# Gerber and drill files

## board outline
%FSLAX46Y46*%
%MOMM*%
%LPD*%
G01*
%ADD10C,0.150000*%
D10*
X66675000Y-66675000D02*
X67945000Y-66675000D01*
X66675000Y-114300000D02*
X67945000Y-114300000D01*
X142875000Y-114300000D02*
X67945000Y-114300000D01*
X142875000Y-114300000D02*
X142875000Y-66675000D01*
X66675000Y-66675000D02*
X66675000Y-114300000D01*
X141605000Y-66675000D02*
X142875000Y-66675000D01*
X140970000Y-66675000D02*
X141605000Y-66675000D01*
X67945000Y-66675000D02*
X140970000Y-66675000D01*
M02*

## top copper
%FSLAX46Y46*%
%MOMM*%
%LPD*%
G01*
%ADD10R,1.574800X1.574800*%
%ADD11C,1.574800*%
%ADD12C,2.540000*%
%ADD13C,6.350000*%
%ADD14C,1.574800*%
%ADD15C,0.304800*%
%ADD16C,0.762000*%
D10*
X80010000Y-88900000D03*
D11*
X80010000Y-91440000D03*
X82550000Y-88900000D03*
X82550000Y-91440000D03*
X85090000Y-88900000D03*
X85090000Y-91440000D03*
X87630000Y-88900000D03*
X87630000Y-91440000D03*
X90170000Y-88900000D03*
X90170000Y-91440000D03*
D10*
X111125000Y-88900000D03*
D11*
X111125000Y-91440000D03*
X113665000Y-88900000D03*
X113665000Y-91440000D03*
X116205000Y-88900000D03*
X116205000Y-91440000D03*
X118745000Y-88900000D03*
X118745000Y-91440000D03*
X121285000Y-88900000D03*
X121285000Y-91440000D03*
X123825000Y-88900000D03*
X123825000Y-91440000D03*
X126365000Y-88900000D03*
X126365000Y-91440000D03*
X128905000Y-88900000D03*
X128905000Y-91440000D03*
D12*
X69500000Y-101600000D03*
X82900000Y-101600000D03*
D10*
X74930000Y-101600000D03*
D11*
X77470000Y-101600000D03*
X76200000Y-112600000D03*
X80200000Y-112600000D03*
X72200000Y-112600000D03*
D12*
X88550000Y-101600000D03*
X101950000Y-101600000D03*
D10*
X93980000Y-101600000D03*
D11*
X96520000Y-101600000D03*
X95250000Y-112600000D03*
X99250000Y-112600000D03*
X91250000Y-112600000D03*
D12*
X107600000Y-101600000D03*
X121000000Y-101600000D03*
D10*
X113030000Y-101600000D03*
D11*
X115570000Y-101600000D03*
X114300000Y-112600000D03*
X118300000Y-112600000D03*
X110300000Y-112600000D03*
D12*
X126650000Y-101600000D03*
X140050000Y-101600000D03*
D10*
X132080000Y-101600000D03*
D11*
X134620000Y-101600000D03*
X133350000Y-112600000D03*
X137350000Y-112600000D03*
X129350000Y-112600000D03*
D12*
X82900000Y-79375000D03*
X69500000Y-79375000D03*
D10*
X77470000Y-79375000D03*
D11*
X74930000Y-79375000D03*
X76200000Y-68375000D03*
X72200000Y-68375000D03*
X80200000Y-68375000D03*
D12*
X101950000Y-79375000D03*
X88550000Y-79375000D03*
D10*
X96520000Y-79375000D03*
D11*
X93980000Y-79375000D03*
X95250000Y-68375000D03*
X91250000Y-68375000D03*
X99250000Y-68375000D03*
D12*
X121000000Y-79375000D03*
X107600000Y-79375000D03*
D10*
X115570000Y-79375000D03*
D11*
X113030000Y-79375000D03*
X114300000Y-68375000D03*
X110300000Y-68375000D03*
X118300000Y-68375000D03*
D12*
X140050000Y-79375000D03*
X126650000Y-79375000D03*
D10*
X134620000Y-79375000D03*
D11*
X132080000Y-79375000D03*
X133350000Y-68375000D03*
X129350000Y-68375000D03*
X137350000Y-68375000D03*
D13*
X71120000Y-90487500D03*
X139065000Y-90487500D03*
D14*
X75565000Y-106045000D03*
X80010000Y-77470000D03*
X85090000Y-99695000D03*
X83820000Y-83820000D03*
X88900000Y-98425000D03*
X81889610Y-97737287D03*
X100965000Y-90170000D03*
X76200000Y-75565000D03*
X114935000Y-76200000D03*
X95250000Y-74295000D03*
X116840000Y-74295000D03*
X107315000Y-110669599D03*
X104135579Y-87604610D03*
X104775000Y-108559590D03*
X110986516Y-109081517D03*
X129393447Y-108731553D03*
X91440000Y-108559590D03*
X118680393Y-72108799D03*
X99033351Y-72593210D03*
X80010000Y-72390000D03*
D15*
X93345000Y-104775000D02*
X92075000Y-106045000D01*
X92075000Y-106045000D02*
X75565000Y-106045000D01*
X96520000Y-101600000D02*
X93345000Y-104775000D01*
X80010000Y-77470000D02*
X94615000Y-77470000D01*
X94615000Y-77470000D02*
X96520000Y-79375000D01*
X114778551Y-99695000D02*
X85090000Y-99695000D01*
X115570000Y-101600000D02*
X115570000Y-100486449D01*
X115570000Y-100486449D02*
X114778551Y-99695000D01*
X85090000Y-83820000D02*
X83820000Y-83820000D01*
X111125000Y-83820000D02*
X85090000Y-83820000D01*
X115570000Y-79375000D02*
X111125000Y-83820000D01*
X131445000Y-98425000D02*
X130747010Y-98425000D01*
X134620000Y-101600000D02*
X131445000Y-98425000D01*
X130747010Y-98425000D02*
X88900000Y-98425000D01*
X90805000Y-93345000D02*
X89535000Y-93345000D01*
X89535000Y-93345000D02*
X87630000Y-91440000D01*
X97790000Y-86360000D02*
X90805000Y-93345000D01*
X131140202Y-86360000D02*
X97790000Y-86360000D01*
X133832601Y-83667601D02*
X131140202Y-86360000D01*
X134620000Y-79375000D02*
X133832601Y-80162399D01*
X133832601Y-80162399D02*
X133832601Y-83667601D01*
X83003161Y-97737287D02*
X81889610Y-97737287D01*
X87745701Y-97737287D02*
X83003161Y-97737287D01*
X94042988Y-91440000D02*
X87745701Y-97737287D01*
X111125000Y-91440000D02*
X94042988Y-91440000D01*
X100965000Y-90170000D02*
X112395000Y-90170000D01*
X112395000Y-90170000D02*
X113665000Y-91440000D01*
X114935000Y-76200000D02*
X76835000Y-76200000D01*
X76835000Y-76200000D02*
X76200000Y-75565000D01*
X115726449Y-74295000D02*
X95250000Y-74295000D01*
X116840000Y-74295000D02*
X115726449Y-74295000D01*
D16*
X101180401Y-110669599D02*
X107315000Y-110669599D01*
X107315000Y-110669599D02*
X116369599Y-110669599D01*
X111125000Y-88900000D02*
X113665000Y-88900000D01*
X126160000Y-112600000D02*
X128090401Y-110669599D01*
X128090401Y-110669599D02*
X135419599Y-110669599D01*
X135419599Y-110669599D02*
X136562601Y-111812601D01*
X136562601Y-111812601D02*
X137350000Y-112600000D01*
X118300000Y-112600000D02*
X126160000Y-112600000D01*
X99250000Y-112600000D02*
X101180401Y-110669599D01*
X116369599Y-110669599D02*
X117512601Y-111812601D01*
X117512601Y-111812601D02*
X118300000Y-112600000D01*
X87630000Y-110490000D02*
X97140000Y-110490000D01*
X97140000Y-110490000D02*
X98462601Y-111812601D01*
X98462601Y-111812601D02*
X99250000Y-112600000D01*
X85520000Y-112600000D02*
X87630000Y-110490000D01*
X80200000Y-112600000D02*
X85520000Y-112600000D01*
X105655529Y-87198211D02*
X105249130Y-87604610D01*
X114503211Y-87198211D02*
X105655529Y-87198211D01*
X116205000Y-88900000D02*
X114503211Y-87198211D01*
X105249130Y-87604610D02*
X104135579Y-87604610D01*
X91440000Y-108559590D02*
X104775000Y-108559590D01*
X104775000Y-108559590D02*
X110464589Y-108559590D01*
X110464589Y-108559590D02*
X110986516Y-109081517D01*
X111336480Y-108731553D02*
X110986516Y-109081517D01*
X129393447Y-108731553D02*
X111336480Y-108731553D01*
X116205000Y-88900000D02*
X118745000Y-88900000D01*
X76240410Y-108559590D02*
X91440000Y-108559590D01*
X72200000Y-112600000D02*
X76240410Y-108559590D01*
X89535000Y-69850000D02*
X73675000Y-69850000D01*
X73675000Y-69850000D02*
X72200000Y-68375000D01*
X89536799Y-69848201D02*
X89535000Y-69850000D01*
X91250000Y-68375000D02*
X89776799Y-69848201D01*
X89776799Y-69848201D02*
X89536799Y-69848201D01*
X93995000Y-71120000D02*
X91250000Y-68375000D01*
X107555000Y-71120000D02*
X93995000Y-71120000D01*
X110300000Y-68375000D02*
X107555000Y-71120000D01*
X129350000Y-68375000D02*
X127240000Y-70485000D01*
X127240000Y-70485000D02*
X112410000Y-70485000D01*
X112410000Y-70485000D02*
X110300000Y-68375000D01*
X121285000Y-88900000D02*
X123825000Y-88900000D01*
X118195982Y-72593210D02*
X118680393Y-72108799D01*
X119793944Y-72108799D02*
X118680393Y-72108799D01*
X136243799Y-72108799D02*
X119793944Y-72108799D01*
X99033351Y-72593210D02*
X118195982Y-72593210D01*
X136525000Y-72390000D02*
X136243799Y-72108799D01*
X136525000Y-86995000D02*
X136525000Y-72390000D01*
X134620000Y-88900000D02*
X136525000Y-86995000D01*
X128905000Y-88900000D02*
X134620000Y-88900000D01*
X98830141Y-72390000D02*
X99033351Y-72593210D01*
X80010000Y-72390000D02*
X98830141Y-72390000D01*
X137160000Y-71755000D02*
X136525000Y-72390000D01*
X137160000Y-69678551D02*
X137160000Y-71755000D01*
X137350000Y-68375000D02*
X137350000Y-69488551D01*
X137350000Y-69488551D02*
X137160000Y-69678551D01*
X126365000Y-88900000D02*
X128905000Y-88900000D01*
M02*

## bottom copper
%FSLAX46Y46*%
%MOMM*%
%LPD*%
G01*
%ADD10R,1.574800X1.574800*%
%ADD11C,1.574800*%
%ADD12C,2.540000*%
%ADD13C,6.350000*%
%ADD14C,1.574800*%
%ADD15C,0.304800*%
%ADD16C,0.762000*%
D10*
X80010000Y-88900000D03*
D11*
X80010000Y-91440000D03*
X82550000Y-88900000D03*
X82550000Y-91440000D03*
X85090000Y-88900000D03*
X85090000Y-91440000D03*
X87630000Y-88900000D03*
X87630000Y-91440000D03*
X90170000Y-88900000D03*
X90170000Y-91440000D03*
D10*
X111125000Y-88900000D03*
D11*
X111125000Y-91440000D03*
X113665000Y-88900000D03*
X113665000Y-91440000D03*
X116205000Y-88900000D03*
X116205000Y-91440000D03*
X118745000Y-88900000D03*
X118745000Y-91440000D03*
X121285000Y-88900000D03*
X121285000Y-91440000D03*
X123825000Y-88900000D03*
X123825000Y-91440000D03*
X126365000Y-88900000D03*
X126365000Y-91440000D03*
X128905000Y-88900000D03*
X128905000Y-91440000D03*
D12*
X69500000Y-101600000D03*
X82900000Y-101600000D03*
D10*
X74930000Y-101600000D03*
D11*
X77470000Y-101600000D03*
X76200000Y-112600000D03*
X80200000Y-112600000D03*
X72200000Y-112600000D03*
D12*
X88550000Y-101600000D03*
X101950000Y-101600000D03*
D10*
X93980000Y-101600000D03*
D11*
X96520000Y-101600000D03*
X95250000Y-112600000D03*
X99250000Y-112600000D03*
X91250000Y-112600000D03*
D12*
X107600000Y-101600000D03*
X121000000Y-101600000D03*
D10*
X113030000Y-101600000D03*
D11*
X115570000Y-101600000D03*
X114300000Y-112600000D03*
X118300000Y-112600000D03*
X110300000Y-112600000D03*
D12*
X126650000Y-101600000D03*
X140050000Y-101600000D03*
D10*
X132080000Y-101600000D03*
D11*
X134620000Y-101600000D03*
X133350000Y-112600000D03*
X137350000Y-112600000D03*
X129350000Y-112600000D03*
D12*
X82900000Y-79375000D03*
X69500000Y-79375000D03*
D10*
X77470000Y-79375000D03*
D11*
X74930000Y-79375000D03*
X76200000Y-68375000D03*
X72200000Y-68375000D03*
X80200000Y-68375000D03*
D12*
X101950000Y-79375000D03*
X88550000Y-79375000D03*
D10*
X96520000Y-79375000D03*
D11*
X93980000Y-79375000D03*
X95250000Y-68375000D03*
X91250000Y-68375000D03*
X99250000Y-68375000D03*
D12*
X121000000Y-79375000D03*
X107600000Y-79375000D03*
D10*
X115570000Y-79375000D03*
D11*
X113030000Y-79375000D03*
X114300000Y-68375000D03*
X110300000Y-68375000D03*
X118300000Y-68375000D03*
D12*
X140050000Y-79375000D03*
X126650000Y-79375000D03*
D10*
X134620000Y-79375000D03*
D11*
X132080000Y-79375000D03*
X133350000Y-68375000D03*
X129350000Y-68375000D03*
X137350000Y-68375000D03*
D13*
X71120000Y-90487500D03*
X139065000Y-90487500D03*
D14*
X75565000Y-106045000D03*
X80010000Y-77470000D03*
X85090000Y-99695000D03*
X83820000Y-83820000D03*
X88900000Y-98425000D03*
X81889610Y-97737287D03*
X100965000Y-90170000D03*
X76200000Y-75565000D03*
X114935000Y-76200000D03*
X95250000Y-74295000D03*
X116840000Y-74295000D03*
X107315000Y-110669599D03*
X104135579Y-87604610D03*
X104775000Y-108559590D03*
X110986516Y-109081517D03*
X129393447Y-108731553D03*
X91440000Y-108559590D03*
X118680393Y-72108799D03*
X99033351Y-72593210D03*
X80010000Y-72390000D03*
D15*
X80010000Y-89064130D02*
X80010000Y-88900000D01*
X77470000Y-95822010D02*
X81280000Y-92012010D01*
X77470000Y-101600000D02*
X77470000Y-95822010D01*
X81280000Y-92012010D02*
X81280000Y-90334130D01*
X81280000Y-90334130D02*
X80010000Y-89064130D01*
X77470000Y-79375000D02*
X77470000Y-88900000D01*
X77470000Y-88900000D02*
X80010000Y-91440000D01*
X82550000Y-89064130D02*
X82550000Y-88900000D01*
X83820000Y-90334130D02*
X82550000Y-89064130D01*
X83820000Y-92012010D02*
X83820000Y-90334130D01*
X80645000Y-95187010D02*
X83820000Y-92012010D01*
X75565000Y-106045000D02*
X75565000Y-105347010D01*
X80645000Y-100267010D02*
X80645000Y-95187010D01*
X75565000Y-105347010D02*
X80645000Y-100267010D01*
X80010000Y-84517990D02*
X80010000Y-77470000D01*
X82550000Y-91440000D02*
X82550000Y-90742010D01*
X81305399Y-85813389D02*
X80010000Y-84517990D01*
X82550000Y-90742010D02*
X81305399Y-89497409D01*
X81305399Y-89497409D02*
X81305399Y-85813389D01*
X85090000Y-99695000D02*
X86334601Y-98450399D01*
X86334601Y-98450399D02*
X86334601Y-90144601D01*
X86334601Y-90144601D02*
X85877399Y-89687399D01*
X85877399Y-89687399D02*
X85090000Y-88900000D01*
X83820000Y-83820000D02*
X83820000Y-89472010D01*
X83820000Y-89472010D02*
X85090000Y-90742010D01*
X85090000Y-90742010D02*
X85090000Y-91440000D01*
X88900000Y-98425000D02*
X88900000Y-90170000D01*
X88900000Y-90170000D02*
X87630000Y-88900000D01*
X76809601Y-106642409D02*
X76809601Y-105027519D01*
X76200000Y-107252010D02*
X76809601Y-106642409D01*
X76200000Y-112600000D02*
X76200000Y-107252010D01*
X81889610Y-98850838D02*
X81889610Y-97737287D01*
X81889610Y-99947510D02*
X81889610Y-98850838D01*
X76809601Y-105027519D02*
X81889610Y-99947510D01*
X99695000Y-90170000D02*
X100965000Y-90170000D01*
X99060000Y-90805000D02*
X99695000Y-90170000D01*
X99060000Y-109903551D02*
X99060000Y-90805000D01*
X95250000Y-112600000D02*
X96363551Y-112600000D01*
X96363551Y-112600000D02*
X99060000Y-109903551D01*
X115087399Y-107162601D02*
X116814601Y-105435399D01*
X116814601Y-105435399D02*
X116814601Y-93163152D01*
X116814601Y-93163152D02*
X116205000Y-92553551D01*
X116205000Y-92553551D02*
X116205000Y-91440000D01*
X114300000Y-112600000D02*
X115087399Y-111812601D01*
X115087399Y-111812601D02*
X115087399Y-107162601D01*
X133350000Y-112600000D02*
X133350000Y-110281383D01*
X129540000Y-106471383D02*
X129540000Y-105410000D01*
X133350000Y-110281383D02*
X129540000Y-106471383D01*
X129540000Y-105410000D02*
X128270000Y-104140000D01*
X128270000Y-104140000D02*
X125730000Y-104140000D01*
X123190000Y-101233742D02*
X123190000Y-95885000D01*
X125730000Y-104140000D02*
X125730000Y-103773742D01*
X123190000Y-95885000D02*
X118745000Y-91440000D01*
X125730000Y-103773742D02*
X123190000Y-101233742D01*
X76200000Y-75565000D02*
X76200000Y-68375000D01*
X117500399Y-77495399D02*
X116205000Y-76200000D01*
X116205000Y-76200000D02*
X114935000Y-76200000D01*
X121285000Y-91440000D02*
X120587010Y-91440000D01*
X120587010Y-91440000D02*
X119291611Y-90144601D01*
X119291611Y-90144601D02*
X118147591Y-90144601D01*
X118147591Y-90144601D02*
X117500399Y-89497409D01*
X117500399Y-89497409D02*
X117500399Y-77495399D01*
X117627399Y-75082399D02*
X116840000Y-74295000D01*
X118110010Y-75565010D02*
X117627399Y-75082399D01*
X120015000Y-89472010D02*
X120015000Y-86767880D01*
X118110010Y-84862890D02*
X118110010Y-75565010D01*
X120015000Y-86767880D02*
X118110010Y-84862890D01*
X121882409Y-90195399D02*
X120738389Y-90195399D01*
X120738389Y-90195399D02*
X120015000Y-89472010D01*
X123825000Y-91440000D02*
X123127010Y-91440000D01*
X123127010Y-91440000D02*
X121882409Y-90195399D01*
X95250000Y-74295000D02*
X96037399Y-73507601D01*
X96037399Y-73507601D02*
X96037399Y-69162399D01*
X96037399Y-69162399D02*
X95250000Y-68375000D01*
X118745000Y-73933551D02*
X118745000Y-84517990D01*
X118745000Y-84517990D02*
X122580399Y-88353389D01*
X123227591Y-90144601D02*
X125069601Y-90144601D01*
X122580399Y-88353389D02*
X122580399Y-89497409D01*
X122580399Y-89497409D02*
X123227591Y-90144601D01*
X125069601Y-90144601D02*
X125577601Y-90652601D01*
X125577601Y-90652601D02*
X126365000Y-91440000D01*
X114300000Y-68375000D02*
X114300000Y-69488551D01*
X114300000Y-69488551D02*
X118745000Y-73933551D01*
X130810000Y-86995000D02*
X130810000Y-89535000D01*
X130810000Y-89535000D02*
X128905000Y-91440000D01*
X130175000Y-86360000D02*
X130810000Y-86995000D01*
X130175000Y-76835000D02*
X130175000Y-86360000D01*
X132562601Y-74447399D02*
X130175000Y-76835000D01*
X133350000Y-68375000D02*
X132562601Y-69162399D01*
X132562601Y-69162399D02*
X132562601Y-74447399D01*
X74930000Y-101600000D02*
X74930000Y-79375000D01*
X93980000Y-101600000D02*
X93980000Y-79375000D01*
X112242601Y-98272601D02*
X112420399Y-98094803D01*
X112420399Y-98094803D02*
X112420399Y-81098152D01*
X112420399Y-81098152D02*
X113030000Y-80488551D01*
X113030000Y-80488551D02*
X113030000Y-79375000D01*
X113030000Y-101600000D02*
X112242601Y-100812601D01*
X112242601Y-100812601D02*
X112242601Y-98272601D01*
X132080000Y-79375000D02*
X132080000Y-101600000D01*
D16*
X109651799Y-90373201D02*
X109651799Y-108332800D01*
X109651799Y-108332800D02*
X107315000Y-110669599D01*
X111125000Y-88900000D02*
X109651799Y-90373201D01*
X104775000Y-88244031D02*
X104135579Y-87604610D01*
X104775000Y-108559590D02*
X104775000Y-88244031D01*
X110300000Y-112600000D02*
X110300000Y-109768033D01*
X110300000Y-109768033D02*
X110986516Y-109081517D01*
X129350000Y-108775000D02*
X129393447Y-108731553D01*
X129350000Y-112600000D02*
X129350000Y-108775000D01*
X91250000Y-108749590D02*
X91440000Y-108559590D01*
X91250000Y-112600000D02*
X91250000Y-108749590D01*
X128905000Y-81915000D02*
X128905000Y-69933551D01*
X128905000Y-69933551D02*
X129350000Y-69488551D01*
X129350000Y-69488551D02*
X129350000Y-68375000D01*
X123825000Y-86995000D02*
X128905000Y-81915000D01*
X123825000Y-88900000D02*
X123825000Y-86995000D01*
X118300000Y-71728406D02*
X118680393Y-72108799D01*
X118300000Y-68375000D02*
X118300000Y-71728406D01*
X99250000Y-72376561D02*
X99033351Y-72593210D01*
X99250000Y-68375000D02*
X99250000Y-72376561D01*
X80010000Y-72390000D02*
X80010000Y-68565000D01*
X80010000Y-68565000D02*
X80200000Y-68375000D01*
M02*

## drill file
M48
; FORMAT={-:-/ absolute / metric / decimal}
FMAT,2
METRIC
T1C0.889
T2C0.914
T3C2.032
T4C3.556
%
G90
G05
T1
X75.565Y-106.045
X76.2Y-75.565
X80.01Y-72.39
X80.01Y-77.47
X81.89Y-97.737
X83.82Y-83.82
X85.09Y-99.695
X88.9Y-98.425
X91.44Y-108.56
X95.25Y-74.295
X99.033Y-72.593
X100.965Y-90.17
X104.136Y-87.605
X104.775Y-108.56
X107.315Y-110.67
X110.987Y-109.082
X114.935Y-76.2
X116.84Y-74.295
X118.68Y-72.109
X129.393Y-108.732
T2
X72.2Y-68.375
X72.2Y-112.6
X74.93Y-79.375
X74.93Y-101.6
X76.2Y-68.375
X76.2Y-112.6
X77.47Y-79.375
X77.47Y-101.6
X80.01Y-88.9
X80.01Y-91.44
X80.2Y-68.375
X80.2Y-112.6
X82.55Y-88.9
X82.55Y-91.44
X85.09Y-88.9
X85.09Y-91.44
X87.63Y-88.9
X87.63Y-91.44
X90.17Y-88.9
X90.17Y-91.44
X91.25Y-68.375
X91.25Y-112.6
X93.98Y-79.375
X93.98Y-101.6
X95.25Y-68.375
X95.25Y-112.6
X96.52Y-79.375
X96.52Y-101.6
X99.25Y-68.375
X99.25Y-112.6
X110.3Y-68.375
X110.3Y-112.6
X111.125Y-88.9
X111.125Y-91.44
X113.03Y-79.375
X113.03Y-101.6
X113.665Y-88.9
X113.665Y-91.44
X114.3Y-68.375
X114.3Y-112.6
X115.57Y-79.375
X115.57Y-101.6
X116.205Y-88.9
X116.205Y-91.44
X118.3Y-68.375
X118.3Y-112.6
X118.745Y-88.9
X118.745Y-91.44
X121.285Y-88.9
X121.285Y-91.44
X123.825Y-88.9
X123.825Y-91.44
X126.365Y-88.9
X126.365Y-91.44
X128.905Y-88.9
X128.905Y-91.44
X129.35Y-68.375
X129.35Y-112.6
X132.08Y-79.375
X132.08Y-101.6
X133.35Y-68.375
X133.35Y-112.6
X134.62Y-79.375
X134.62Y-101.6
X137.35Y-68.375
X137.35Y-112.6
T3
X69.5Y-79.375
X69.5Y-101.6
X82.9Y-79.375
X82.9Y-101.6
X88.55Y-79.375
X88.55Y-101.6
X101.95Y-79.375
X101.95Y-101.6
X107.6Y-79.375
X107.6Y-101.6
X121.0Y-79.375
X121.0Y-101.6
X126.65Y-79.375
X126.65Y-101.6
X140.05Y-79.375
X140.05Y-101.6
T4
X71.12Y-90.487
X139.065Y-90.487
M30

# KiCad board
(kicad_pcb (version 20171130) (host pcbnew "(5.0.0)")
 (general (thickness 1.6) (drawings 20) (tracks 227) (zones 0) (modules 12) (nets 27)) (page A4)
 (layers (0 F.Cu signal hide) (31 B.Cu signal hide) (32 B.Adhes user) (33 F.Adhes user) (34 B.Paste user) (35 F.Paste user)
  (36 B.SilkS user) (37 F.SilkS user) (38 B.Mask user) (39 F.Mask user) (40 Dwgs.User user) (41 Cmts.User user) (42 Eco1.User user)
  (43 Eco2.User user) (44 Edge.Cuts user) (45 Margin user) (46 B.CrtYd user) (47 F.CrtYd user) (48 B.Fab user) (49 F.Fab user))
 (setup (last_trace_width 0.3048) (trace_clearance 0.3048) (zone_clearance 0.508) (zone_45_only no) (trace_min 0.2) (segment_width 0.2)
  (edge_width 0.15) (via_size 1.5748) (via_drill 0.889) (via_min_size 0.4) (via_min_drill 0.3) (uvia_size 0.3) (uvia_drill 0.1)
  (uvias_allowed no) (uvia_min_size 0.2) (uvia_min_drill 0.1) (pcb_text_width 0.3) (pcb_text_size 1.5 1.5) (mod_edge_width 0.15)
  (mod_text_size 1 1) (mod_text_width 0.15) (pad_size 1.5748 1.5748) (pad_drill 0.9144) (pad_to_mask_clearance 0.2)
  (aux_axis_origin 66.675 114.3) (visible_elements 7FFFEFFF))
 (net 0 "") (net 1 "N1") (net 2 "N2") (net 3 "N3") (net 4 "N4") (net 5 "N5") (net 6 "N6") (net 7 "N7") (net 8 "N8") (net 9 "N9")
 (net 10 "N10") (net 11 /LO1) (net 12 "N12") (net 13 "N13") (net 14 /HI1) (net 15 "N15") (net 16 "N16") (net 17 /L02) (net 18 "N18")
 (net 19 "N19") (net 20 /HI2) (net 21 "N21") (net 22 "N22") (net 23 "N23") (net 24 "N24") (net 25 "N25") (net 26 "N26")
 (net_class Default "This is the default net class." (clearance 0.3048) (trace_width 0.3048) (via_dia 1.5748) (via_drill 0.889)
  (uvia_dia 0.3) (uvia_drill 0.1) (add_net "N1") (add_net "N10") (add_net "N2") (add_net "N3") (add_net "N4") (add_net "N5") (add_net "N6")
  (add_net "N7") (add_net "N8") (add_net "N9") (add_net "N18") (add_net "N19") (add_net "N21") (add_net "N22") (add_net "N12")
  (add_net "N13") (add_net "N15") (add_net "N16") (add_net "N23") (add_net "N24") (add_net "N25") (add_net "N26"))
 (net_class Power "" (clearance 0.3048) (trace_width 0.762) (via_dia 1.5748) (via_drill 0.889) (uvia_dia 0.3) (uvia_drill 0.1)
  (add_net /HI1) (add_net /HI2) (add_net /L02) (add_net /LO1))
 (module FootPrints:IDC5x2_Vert (layer B.Cu) (at 85.09 90.17 180)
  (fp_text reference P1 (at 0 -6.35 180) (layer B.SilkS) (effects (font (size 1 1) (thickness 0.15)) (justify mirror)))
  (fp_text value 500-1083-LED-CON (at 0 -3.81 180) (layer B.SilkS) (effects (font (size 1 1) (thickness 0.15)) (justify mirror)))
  (pad 1 thru_hole rect (at 5.08 1.27 180) (size 1.5748 1.5748) (drill 0.9144) (layers *.Cu *.Mask B.SilkS) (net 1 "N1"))
  (pad 2 thru_hole circle (at 5.08 -1.27 180) (size 1.5748 1.5748) (drill 0.9144) (layers *.Cu *.Mask B.SilkS) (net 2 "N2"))
  (pad 3 thru_hole circle (at 2.54 1.27 180) (size 1.5748 1.5748) (drill 0.9144) (layers *.Cu *.Mask B.SilkS) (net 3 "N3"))
  (pad 4 thru_hole circle (at 2.54 -1.27 180) (size 1.5748 1.5748) (drill 0.9144) (layers *.Cu *.Mask B.SilkS) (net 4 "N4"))
  (pad 5 thru_hole circle (at 0 1.27 180) (size 1.5748 1.5748) (drill 0.9144) (layers *.Cu *.Mask B.SilkS) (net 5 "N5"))
  (pad 6 thru_hole circle (at 0 -1.27 180) (size 1.5748 1.5748) (drill 0.9144) (layers *.Cu *.Mask B.SilkS) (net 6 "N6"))
  (pad 7 thru_hole circle (at -2.54 1.27 180) (size 1.5748 1.5748) (drill 0.9144) (layers *.Cu *.Mask B.SilkS) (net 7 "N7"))
  (pad 8 thru_hole circle (at -2.54 -1.27 180) (size 1.5748 1.5748) (drill 0.9144) (layers *.Cu *.Mask B.SilkS) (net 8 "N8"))
  (pad 9 thru_hole circle (at -5.08 1.27 180) (size 1.5748 1.5748) (drill 0.9144) (layers *.Cu *.Mask B.SilkS) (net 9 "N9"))
  (pad 10 thru_hole circle (at -5.08 -1.27 180) (size 1.5748 1.5748) (drill 0.9144) (layers *.Cu *.Mask B.SilkS) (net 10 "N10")))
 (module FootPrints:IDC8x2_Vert (layer B.Cu) (at 120.015 90.17 180)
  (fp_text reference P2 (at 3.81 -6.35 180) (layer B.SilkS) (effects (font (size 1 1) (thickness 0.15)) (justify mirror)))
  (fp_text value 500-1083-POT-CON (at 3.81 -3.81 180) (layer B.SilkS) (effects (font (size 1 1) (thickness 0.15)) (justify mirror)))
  (pad 1 thru_hole rect (at 8.89 1.27 180) (size 1.5748 1.5748) (drill 0.9144) (layers *.Cu *.Mask B.SilkS) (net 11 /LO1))
  (pad 2 thru_hole circle (at 8.89 -1.27 180) (size 1.5748 1.5748) (drill 0.9144) (layers *.Cu *.Mask B.SilkS) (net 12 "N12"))
  (pad 3 thru_hole circle (at 6.35 1.27 180) (size 1.5748 1.5748) (drill 0.9144) (layers *.Cu *.Mask B.SilkS) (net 11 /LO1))
  (pad 4 thru_hole circle (at 6.35 -1.27 180) (size 1.5748 1.5748) (drill 0.9144) (layers *.Cu *.Mask B.SilkS) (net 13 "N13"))
  (pad 5 thru_hole circle (at 3.81 1.27 180) (size 1.5748 1.5748) (drill 0.9144) (layers *.Cu *.Mask B.SilkS) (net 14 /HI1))
  (pad 6 thru_hole circle (at 3.81 -1.27 180) (size 1.5748 1.5748) (drill 0.9144) (layers *.Cu *.Mask B.SilkS) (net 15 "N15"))
  (pad 7 thru_hole circle (at 1.27 1.27 180) (size 1.5748 1.5748) (drill 0.9144) (layers *.Cu *.Mask B.SilkS) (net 14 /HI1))
  (pad 8 thru_hole circle (at 1.27 -1.27 180) (size 1.5748 1.5748) (drill 0.9144) (layers *.Cu *.Mask B.SilkS) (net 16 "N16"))
  (pad 9 thru_hole circle (at -1.27 1.27 180) (size 1.5748 1.5748) (drill 0.9144) (layers *.Cu *.Mask B.SilkS) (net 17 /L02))
  (pad 10 thru_hole circle (at -1.27 -1.27 180) (size 1.5748 1.5748) (drill 0.9144) (layers *.Cu *.Mask B.SilkS) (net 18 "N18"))
  (pad 11 thru_hole circle (at -3.81 1.27 180) (size 1.5748 1.5748) (drill 0.9144) (layers *.Cu *.Mask B.SilkS) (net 17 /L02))
  (pad 12 thru_hole circle (at -3.81 -1.27 180) (size 1.5748 1.5748) (drill 0.9144) (layers *.Cu *.Mask B.SilkS) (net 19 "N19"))
  (pad 13 thru_hole circle (at -6.35 1.27 180) (size 1.5748 1.5748) (drill 0.9144) (layers *.Cu *.Mask B.SilkS) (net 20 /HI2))
  (pad 14 thru_hole circle (at -6.35 -1.27 180) (size 1.5748 1.5748) (drill 0.9144) (layers *.Cu *.Mask B.SilkS) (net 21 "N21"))
  (pad 15 thru_hole circle (at -8.89 1.27 180) (size 1.5748 1.5748) (drill 0.9144) (layers *.Cu *.Mask B.SilkS) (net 20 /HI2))
  (pad 16 thru_hole circle (at -8.89 -1.27 180) (size 1.5748 1.5748) (drill 0.9144) (layers *.Cu *.Mask B.SilkS) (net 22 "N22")))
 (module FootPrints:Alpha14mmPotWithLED (layer F.Cu) (at 76.2 101.6)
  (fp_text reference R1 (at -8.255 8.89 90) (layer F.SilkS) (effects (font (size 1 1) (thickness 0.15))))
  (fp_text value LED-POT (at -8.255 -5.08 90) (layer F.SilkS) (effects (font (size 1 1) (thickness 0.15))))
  (pad "" thru_hole circle (at -6.7 0) (size 2.54 2.54) (drill 2.032) (layers *.Cu *.Mask F.SilkS))
  (pad "" thru_hole circle (at 6.7 0) (size 2.54 2.54) (drill 2.032) (layers *.Cu *.Mask F.SilkS))
  (pad 4 thru_hole rect (at -1.27 0) (size 1.5748 1.5748) (drill 0.9144) (layers *.Cu *.Mask F.SilkS) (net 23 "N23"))
  (pad 5 thru_hole circle (at 1.27 0) (size 1.5748 1.5748) (drill 0.9144) (layers *.Cu *.Mask F.SilkS) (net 1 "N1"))
  (pad 2 thru_hole circle (at 0 11) (size 1.5748 1.5748) (drill 0.9144) (layers *.Cu *.Mask F.SilkS) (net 12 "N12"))
  (pad 3 thru_hole circle (at 4 11) (size 1.5748 1.5748) (drill 0.9144) (layers *.Cu *.Mask F.SilkS) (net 11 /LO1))
  (pad 1 thru_hole circle (at -4 11) (size 1.5748 1.5748) (drill 0.9144) (layers *.Cu *.Mask F.SilkS) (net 14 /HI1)))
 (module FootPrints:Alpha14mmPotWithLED (layer F.Cu) (at 95.25 101.6)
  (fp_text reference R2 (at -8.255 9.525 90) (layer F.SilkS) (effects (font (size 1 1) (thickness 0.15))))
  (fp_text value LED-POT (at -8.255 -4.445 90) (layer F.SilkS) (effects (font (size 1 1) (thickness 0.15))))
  (pad "" thru_hole circle (at -6.7 0) (size 2.54 2.54) (drill 2.032) (layers *.Cu *.Mask F.SilkS))
  (pad "" thru_hole circle (at 6.7 0) (size 2.54 2.54) (drill 2.032) (layers *.Cu *.Mask F.SilkS))
  (pad 4 thru_hole rect (at -1.27 0) (size 1.5748 1.5748) (drill 0.9144) (layers *.Cu *.Mask F.SilkS) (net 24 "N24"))
  (pad 5 thru_hole circle (at 1.27 0) (size 1.5748 1.5748) (drill 0.9144) (layers *.Cu *.Mask F.SilkS) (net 3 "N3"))
  (pad 2 thru_hole circle (at 0 11) (size 1.5748 1.5748) (drill 0.9144) (layers *.Cu *.Mask F.SilkS) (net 13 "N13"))
  (pad 3 thru_hole circle (at 4 11) (size 1.5748 1.5748) (drill 0.9144) (layers *.Cu *.Mask F.SilkS) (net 11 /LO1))
  (pad 1 thru_hole circle (at -4 11) (size 1.5748 1.5748) (drill 0.9144) (layers *.Cu *.Mask F.SilkS) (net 14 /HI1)))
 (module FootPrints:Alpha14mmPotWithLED (layer F.Cu) (at 114.3 101.6)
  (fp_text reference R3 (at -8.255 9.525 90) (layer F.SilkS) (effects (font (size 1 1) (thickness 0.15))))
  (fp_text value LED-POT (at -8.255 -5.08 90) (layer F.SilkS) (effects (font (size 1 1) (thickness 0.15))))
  (pad "" thru_hole circle (at -6.7 0) (size 2.54 2.54) (drill 2.032) (layers *.Cu *.Mask F.SilkS))
  (pad "" thru_hole circle (at 6.7 0) (size 2.54 2.54) (drill 2.032) (layers *.Cu *.Mask F.SilkS))
  (pad 4 thru_hole rect (at -1.27 0) (size 1.5748 1.5748) (drill 0.9144) (layers *.Cu *.Mask F.SilkS) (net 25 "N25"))
  (pad 5 thru_hole circle (at 1.27 0) (size 1.5748 1.5748) (drill 0.9144) (layers *.Cu *.Mask F.SilkS) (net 5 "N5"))
  (pad 2 thru_hole circle (at 0 11) (size 1.5748 1.5748) (drill 0.9144) (layers *.Cu *.Mask F.SilkS) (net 15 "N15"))
  (pad 3 thru_hole circle (at 4 11) (size 1.5748 1.5748) (drill 0.9144) (layers *.Cu *.Mask F.SilkS) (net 11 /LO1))
  (pad 1 thru_hole circle (at -4 11) (size 1.5748 1.5748) (drill 0.9144) (layers *.Cu *.Mask F.SilkS) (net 14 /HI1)))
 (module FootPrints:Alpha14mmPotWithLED (layer F.Cu) (at 133.35 101.6)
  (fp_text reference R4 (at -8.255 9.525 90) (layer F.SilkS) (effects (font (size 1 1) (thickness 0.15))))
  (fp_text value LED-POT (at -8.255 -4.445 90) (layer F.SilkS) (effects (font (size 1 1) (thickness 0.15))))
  (pad "" thru_hole circle (at -6.7 0) (size 2.54 2.54) (drill 2.032) (layers *.Cu *.Mask F.SilkS))
  (pad "" thru_hole circle (at 6.7 0) (size 2.54 2.54) (drill 2.032) (layers *.Cu *.Mask F.SilkS))
  (pad 4 thru_hole rect (at -1.27 0) (size 1.5748 1.5748) (drill 0.9144) (layers *.Cu *.Mask F.SilkS) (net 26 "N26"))
  (pad 5 thru_hole circle (at 1.27 0) (size 1.5748 1.5748) (drill 0.9144) (layers *.Cu *.Mask F.SilkS) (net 7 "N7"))
  (pad 2 thru_hole circle (at 0 11) (size 1.5748 1.5748) (drill 0.9144) (layers *.Cu *.Mask F.SilkS) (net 16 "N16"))
  (pad 3 thru_hole circle (at 4 11) (size 1.5748 1.5748) (drill 0.9144) (layers *.Cu *.Mask F.SilkS) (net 11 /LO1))
  (pad 1 thru_hole circle (at -4 11) (size 1.5748 1.5748) (drill 0.9144) (layers *.Cu *.Mask F.SilkS) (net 14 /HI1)))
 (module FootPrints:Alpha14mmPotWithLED (layer F.Cu) (at 76.2 79.375 180)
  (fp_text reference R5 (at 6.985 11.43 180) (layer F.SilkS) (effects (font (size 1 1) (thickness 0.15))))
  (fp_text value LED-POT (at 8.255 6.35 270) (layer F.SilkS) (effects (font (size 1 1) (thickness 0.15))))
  (pad "" thru_hole circle (at -6.7 0 180) (size 2.54 2.54) (drill 2.032) (layers *.Cu *.Mask F.SilkS))
  (pad "" thru_hole circle (at 6.7 0 180) (size 2.54 2.54) (drill 2.032) (layers *.Cu *.Mask F.SilkS))
  (pad 4 thru_hole rect (at -1.27 0 180) (size 1.5748 1.5748) (drill 0.9144) (layers *.Cu *.Mask F.SilkS) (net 2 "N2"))
  (pad 5 thru_hole circle (at 1.27 0 180) (size 1.5748 1.5748) (drill 0.9144) (layers *.Cu *.Mask F.SilkS) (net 23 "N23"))
  (pad 2 thru_hole circle (at 0 11 180) (size 1.5748 1.5748) (drill 0.9144) (layers *.Cu *.Mask F.SilkS) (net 18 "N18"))
  (pad 3 thru_hole circle (at 4 11 180) (size 1.5748 1.5748) (drill 0.9144) (layers *.Cu *.Mask F.SilkS) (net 17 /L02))
  (pad 1 thru_hole circle (at -4 11 180) (size 1.5748 1.5748) (drill 0.9144) (layers *.Cu *.Mask F.SilkS) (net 20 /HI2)))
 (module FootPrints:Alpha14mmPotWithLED (layer F.Cu) (at 95.25 79.375 180)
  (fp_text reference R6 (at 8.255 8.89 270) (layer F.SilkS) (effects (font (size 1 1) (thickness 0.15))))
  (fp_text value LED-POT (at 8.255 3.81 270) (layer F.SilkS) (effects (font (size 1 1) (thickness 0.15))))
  (pad "" thru_hole circle (at -6.7 0 180) (size 2.54 2.54) (drill 2.032) (layers *.Cu *.Mask F.SilkS))
  (pad "" thru_hole circle (at 6.7 0 180) (size 2.54 2.54) (drill 2.032) (layers *.Cu *.Mask F.SilkS))
  (pad 4 thru_hole rect (at -1.27 0 180) (size 1.5748 1.5748) (drill 0.9144) (layers *.Cu *.Mask F.SilkS) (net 4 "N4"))
  (pad 5 thru_hole circle (at 1.27 0 180) (size 1.5748 1.5748) (drill 0.9144) (layers *.Cu *.Mask F.SilkS) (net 24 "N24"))
  (pad 2 thru_hole circle (at 0 11 180) (size 1.5748 1.5748) (drill 0.9144) (layers *.Cu *.Mask F.SilkS) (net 19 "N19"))
  (pad 3 thru_hole circle (at 4 11 180) (size 1.5748 1.5748) (drill 0.9144) (layers *.Cu *.Mask F.SilkS) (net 17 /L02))
  (pad 1 thru_hole circle (at -4 11 180) (size 1.5748 1.5748) (drill 0.9144) (layers *.Cu *.Mask F.SilkS) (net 20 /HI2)))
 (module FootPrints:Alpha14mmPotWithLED (layer F.Cu) (at 114.3 79.375 180)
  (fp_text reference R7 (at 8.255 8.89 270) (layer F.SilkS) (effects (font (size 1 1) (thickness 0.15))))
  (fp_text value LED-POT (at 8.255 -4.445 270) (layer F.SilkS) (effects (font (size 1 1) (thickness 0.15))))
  (pad "" thru_hole circle (at -6.7 0 180) (size 2.54 2.54) (drill 2.032) (layers *.Cu *.Mask F.SilkS))
  (pad "" thru_hole circle (at 6.7 0 180) (size 2.54 2.54) (drill 2.032) (layers *.Cu *.Mask F.SilkS))
  (pad 4 thru_hole rect (at -1.27 0 180) (size 1.5748 1.5748) (drill 0.9144) (layers *.Cu *.Mask F.SilkS) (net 6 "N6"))
  (pad 5 thru_hole circle (at 1.27 0 180) (size 1.5748 1.5748) (drill 0.9144) (layers *.Cu *.Mask F.SilkS) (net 25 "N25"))
  (pad 2 thru_hole circle (at 0 11 180) (size 1.5748 1.5748) (drill 0.9144) (layers *.Cu *.Mask F.SilkS) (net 21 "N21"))
  (pad 3 thru_hole circle (at 4 11 180) (size 1.5748 1.5748) (drill 0.9144) (layers *.Cu *.Mask F.SilkS) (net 17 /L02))
  (pad 1 thru_hole circle (at -4 11 180) (size 1.5748 1.5748) (drill 0.9144) (layers *.Cu *.Mask F.SilkS) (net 20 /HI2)))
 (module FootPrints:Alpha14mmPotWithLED (layer F.Cu) (at 133.35 79.375 180)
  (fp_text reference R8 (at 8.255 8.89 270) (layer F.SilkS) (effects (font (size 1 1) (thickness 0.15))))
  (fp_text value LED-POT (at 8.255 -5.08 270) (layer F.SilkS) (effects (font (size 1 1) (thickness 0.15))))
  (pad "" thru_hole circle (at -6.7 0 180) (size 2.54 2.54) (drill 2.032) (layers *.Cu *.Mask F.SilkS))
  (pad "" thru_hole circle (at 6.7 0 180) (size 2.54 2.54) (drill 2.032) (layers *.Cu *.Mask F.SilkS))
  (pad 4 thru_hole rect (at -1.27 0 180) (size 1.5748 1.5748) (drill 0.9144) (layers *.Cu *.Mask F.SilkS) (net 8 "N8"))
  (pad 5 thru_hole circle (at 1.27 0 180) (size 1.5748 1.5748) (drill 0.9144) (layers *.Cu *.Mask F.SilkS) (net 26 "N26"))
  (pad 2 thru_hole circle (at 0 11 180) (size 1.5748 1.5748) (drill 0.9144) (layers *.Cu *.Mask F.SilkS) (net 22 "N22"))
  (pad 3 thru_hole circle (at 4 11 180) (size 1.5748 1.5748) (drill 0.9144) (layers *.Cu *.Mask F.SilkS) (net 17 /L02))
  (pad 1 thru_hole circle (at -4 11 180) (size 1.5748 1.5748) (drill 0.9144) (layers *.Cu *.Mask F.SilkS) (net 20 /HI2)))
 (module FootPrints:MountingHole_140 (layer F.Cu) (at 71.12 90.805)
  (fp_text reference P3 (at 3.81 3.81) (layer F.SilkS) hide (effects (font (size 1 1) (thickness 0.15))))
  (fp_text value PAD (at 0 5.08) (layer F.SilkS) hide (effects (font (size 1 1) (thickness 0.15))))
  (pad "" thru_hole circle (at 0 -0.3175) (size 6.35 6.35) (drill 3.556) (layers *.Cu *.Mask F.SilkS)))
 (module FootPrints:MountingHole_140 (layer F.Cu) (at 139.065 90.17)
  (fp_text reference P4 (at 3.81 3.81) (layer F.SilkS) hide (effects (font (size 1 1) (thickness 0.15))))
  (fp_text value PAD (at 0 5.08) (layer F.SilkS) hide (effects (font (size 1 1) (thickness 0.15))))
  (pad "" thru_hole circle (at 0 0.3175) (size 6.35 6.35) (drill 3.556) (layers *.Cu *.Mask F.SilkS)))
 (gr_line (start 66.675 66.675) (end 67.945 66.675) (angle 90) (layer Edge.Cuts) (width 0.15))
 (gr_line (start 66.675 114.3) (end 67.945 114.3) (angle 90) (layer Edge.Cuts) (width 0.15))
 (gr_line (start 142.875 114.3) (end 67.945 114.3) (angle 90) (layer Edge.Cuts) (width 0.15))
 (gr_line (start 142.875 114.3) (end 142.875 66.675) (angle 90) (layer Edge.Cuts) (width 0.15))
 (gr_line (start 66.675 66.675) (end 66.675 114.3) (angle 90) (layer Edge.Cuts) (width 0.15))
 (gr_line (start 141.605 66.675) (end 142.875 66.675) (angle 90) (layer Edge.Cuts) (width 0.15))
 (gr_line (start 140.97 66.675) (end 141.605 66.675) (angle 90) (layer Edge.Cuts) (width 0.15))
 (gr_line (start 67.945 66.675) (end 140.97 66.675) (angle 90) (layer Edge.Cuts) (width 0.15))
 (segment (start 80.01 89.06413) (end 80.01 88.9) (width 0.3048) (layer B.Cu) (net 1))
 (segment (start 77.47 95.82201) (end 81.28 92.01201) (width 0.3048) (layer B.Cu) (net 1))
 (segment (start 77.47 101.6) (end 77.47 95.82201) (width 0.3048) (layer B.Cu) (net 1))
 (segment (start 81.28 92.01201) (end 81.28 90.33413) (width 0.3048) (layer B.Cu) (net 1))
 (segment (start 81.28 90.33413) (end 80.01 89.06413) (width 0.3048) (layer B.Cu) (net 1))
 (segment (start 77.47 79.375) (end 77.47 88.9) (width 0.3048) (layer B.Cu) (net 2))
 (segment (start 77.47 88.9) (end 80.01 91.44) (width 0.3048) (layer B.Cu) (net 2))
 (segment (start 82.55 89.06413) (end 82.55 88.9) (width 0.3048) (layer B.Cu) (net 3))
 (segment (start 83.82 90.33413) (end 82.55 89.06413) (width 0.3048) (layer B.Cu) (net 3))
 (segment (start 83.82 92.01201) (end 83.82 90.33413) (width 0.3048) (layer B.Cu) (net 3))
 (segment (start 80.645 95.18701) (end 83.82 92.01201) (width 0.3048) (layer B.Cu) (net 3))
 (segment (start 75.565 106.045) (end 75.565 105.34701) (width 0.3048) (layer B.Cu) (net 3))
 (segment (start 80.645 100.26701) (end 80.645 95.18701) (width 0.3048) (layer B.Cu) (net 3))
 (segment (start 75.565 105.34701) (end 80.645 100.26701) (width 0.3048) (layer B.Cu) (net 3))
 (segment (start 93.345 104.775) (end 92.075 106.045) (width 0.3048) (layer F.Cu) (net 3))
 (segment (start 92.075 106.045) (end 75.565 106.045) (width 0.3048) (layer F.Cu) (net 3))
 (via (at 75.565 106.045) (size 1.5748) (drill 0.889) (layers F.Cu B.Cu) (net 3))
 (segment (start 96.52 101.6) (end 93.345 104.775) (width 0.3048) (layer F.Cu) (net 3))
 (segment (start 80.01 77.47) (end 94.615 77.47) (width 0.3048) (layer F.Cu) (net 4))
 (segment (start 94.615 77.47) (end 96.52 79.375) (width 0.3048) (layer F.Cu) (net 4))
 (via (at 80.01 77.47) (size 1.5748) (drill 0.889) (layers F.Cu B.Cu) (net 4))
 (segment (start 80.01 84.51799) (end 80.01 77.47) (width 0.3048) (layer B.Cu) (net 4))
 (segment (start 82.55 91.44) (end 82.55 90.74201) (width 0.3048) (layer B.Cu) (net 4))
 (segment (start 81.305399 85.813389) (end 80.01 84.51799) (width 0.3048) (layer B.Cu) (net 4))
 (segment (start 82.55 90.74201) (end 81.305399 89.497409) (width 0.3048) (layer B.Cu) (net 4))
 (segment (start 81.305399 89.497409) (end 81.305399 85.813389) (width 0.3048) (layer B.Cu) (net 4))
 (segment (start 85.09 99.695) (end 86.334601 98.450399) (width 0.3048) (layer B.Cu) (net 5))
 (segment (start 86.334601 98.450399) (end 86.334601 90.144601) (width 0.3048) (layer B.Cu) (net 5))
 (segment (start 86.334601 90.144601) (end 85.877399 89.687399) (width 0.3048) (layer B.Cu) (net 5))
 (segment (start 85.877399 89.687399) (end 85.09 88.9) (width 0.3048) (layer B.Cu) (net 5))
 (segment (start 114.778551 99.695) (end 85.09 99.695) (width 0.3048) (layer F.Cu) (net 5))
 (via (at 85.09 99.695) (size 1.5748) (drill 0.889) (layers F.Cu B.Cu) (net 5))
 (segment (start 115.57 101.6) (end 115.57 100.486449) (width 0.3048) (layer F.Cu) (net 5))
 (segment (start 115.57 100.486449) (end 114.778551 99.695) (width 0.3048) (layer F.Cu) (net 5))
 (segment (start 83.82 83.82) (end 83.82 89.47201) (width 0.3048) (layer B.Cu) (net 6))
 (segment (start 83.82 89.47201) (end 85.09 90.74201) (width 0.3048) (layer B.Cu) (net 6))
 (segment (start 85.09 90.74201) (end 85.09 91.44) (width 0.3048) (layer B.Cu) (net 6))
 (segment (start 85.09 83.82) (end 83.82 83.82) (width 0.3048) (layer F.Cu) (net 6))
 (via (at 83.82 83.82) (size 1.5748) (drill 0.889) (layers F.Cu B.Cu) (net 6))
 (segment (start 111.125 83.82) (end 85.09 83.82) (width 0.3048) (layer F.Cu) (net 6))
 (segment (start 115.57 79.375) (end 111.125 83.82) (width 0.3048) (layer F.Cu) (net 6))
 (segment (start 88.9 98.425) (end 88.9 90.17) (width 0.3048) (layer B.Cu) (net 7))
 (segment (start 88.9 90.17) (end 87.63 88.9) (width 0.3048) (layer B.Cu) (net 7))
 (segment (start 131.445 98.425) (end 130.74701 98.425) (width 0.3048) (layer F.Cu) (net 7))
 (via (at 88.9 98.425) (size 1.5748) (drill 0.889) (layers F.Cu B.Cu) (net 7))
 (segment (start 134.62 101.6) (end 131.445 98.425) (width 0.3048) (layer F.Cu) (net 7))
 (segment (start 130.74701 98.425) (end 88.9 98.425) (width 0.3048) (layer F.Cu) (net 7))
 (segment (start 90.805 93.345) (end 89.535 93.345) (width 0.3048) (layer F.Cu) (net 8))
 (segment (start 89.535 93.345) (end 87.63 91.44) (width 0.3048) (layer F.Cu) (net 8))
 (segment (start 97.79 86.36) (end 90.805 93.345) (width 0.3048) (layer F.Cu) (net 8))
 (segment (start 131.140202 86.36) (end 97.79 86.36) (width 0.3048) (layer F.Cu) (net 8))
 (segment (start 133.832601 83.667601) (end 131.140202 86.36) (width 0.3048) (layer F.Cu) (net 8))
 (segment (start 134.62 79.375) (end 133.832601 80.162399) (width 0.3048) (layer F.Cu) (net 8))
 (segment (start 133.832601 80.162399) (end 133.832601 83.667601) (width 0.3048) (layer F.Cu) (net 8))
 (segment (start 83.003161 97.737287) (end 81.88961 97.737287) (width 0.3048) (layer F.Cu) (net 12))
 (segment (start 87.745701 97.737287) (end 83.003161 97.737287) (width 0.3048) (layer F.Cu) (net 12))
 (segment (start 94.042988 91.44) (end 87.745701 97.737287) (width 0.3048) (layer F.Cu) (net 12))
 (segment (start 111.125 91.44) (end 94.042988 91.44) (width 0.3048) (layer F.Cu) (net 12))
 (segment (start 76.809601 106.642409) (end 76.809601 105.027519) (width 0.3048) (layer B.Cu) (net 12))
 (segment (start 76.2 107.25201) (end 76.809601 106.642409) (width 0.3048) (layer B.Cu) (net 12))
 (segment (start 76.2 112.6) (end 76.2 107.25201) (width 0.3048) (layer B.Cu) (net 12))
 (segment (start 81.88961 98.850838) (end 81.88961 97.737287) (width 0.3048) (layer B.Cu) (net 12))
 (via (at 81.88961 97.737287) (size 1.5748) (drill 0.889) (layers F.Cu B.Cu) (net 12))
 (segment (start 81.88961 99.94751) (end 81.88961 98.850838) (width 0.3048) (layer B.Cu) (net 12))
 (segment (start 76.809601 105.027519) (end 81.88961 99.94751) (width 0.3048) (layer B.Cu) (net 12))
 (segment (start 100.965 90.17) (end 112.395 90.17) (width 0.3048) (layer F.Cu) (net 13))
 (segment (start 112.395 90.17) (end 113.665 91.44) (width 0.3048) (layer F.Cu) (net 13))
 (segment (start 99.695 90.17) (end 100.965 90.17) (width 0.3048) (layer B.Cu) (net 13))
 (via (at 100.965 90.17) (size 1.5748) (drill 0.889) (layers F.Cu B.Cu) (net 13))
 (segment (start 99.06 90.805) (end 99.695 90.17) (width 0.3048) (layer B.Cu) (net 13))
 (segment (start 99.06 109.903551) (end 99.06 90.805) (width 0.3048) (layer B.Cu) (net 13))
 (segment (start 95.25 112.6) (end 96.363551 112.6) (width 0.3048) (layer B.Cu) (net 13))
 (segment (start 96.363551 112.6) (end 99.06 109.903551) (width 0.3048) (layer B.Cu) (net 13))
 (segment (start 115.087399 107.162601) (end 116.814601 105.435399) (width 0.3048) (layer B.Cu) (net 15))
 (segment (start 116.814601 105.435399) (end 116.814601 93.163152) (width 0.3048) (layer B.Cu) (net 15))
 (segment (start 116.814601 93.163152) (end 116.205 92.553551) (width 0.3048) (layer B.Cu) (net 15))
 (segment (start 116.205 92.553551) (end 116.205 91.44) (width 0.3048) (layer B.Cu) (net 15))
 (segment (start 114.3 112.6) (end 115.087399 111.812601) (width 0.3048) (layer B.Cu) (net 15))
 (segment (start 115.087399 111.812601) (end 115.087399 107.162601) (width 0.3048) (layer B.Cu) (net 15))
 (segment (start 133.35 112.6) (end 133.35 110.281383) (width 0.3048) (layer B.Cu) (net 16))
 (segment (start 129.54 106.471383) (end 129.54 105.41) (width 0.3048) (layer B.Cu) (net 16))
 (segment (start 133.35 110.281383) (end 129.54 106.471383) (width 0.3048) (layer B.Cu) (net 16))
 (segment (start 129.54 105.41) (end 128.27 104.14) (width 0.3048) (layer B.Cu) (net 16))
 (segment (start 128.27 104.14) (end 125.73 104.14) (width 0.3048) (layer B.Cu) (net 16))
 (segment (start 123.19 101.233742) (end 123.19 95.885) (width 0.3048) (layer B.Cu) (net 16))
 (segment (start 125.73 104.14) (end 125.73 103.773742) (width 0.3048) (layer B.Cu) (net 16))
 (segment (start 123.19 95.885) (end 118.745 91.44) (width 0.3048) (layer B.Cu) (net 16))
 (segment (start 125.73 103.773742) (end 123.19 101.233742) (width 0.3048) (layer B.Cu) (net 16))
 (segment (start 76.2 75.565) (end 76.2 68.375) (width 0.3048) (layer B.Cu) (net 18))
 (segment (start 114.935 76.2) (end 76.835 76.2) (width 0.3048) (layer F.Cu) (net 18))
 (via (at 76.2 75.565) (size 1.5748) (drill 0.889) (layers F.Cu B.Cu) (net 18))
 (segment (start 76.835 76.2) (end 76.2 75.565) (width 0.3048) (layer F.Cu) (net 18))
 (segment (start 117.500399 77.495399) (end 116.205 76.2) (width 0.3048) (layer B.Cu) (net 18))
 (segment (start 116.205 76.2) (end 114.935 76.2) (width 0.3048) (layer B.Cu) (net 18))
 (via (at 114.935 76.2) (size 1.5748) (drill 0.889) (layers F.Cu B.Cu) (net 18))
 (segment (start 121.285 91.44) (end 120.58701 91.44) (width 0.3048) (layer B.Cu) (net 18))
 (segment (start 120.58701 91.44) (end 119.291611 90.144601) (width 0.3048) (layer B.Cu) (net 18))
 (segment (start 119.291611 90.144601) (end 118.147591 90.144601) (width 0.3048) (layer B.Cu) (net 18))
 (segment (start 118.147591 90.144601) (end 117.500399 89.497409) (width 0.3048) (layer B.Cu) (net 18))
 (segment (start 117.500399 89.497409) (end 117.500399 77.495399) (width 0.3048) (layer B.Cu) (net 18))
 (segment (start 117.627399 75.082399) (end 116.84 74.295) (width 0.3048) (layer B.Cu) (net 19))
 (segment (start 118.11001 75.56501) (end 117.627399 75.082399) (width 0.3048) (layer B.Cu) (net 19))
 (segment (start 120.015 89.47201) (end 120.015 86.76788) (width 0.3048) (layer B.Cu) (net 19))
 (segment (start 118.11001 84.86289) (end 118.11001 75.56501) (width 0.3048) (layer B.Cu) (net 19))
 (segment (start 120.015 86.76788) (end 118.11001 84.86289) (width 0.3048) (layer B.Cu) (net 19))
 (segment (start 121.882409 90.195399) (end 120.738389 90.195399) (width 0.3048) (layer B.Cu) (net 19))
 (segment (start 120.738389 90.195399) (end 120.015 89.47201) (width 0.3048) (layer B.Cu) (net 19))
 (segment (start 123.825 91.44) (end 123.12701 91.44) (width 0.3048) (layer B.Cu) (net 19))
 (segment (start 123.12701 91.44) (end 121.882409 90.195399) (width 0.3048) (layer B.Cu) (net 19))
 (segment (start 95.25 74.295) (end 96.037399 73.507601) (width 0.3048) (layer B.Cu) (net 19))
 (segment (start 96.037399 73.507601) (end 96.037399 69.162399) (width 0.3048) (layer B.Cu) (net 19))
 (segment (start 96.037399 69.162399) (end 95.25 68.375) (width 0.3048) (layer B.Cu) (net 19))
 (segment (start 115.726449 74.295) (end 95.25 74.295) (width 0.3048) (layer F.Cu) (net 19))
 (via (at 95.25 74.295) (size 1.5748) (drill 0.889) (layers F.Cu B.Cu) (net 19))
 (segment (start 116.84 74.295) (end 115.726449 74.295) (width 0.3048) (layer F.Cu) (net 19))
 (via (at 116.84 74.295) (size 1.5748) (drill 0.889) (layers F.Cu B.Cu) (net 19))
 (segment (start 118.745 73.933551) (end 118.745 84.51799) (width 0.3048) (layer B.Cu) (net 21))
 (segment (start 118.745 84.51799) (end 122.580399 88.353389) (width 0.3048) (layer B.Cu) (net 21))
 (segment (start 123.227591 90.144601) (end 125.069601 90.144601) (width 0.3048) (layer B.Cu) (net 21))
 (segment (start 122.580399 88.353389) (end 122.580399 89.497409) (width 0.3048) (layer B.Cu) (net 21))
 (segment (start 122.580399 89.497409) (end 123.227591 90.144601) (width 0.3048) (layer B.Cu) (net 21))
 (segment (start 125.069601 90.144601) (end 125.577601 90.652601) (width 0.3048) (layer B.Cu) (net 21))
 (segment (start 125.577601 90.652601) (end 126.365 91.44) (width 0.3048) (layer B.Cu) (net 21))
 (segment (start 114.3 68.375) (end 114.3 69.488551) (width 0.3048) (layer B.Cu) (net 21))
 (segment (start 114.3 69.488551) (end 118.745 73.933551) (width 0.3048) (layer B.Cu) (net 21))
 (segment (start 130.81 86.995) (end 130.81 89.535) (width 0.3048) (layer B.Cu) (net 22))
 (segment (start 130.81 89.535) (end 128.905 91.44) (width 0.3048) (layer B.Cu) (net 22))
 (segment (start 130.175 86.36) (end 130.81 86.995) (width 0.3048) (layer B.Cu) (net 22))
 (segment (start 130.175 76.835) (end 130.175 86.36) (width 0.3048) (layer B.Cu) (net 22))
 (segment (start 132.562601 74.447399) (end 130.175 76.835) (width 0.3048) (layer B.Cu) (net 22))
 (segment (start 133.35 68.375) (end 132.562601 69.162399) (width 0.3048) (layer B.Cu) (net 22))
 (segment (start 132.562601 69.162399) (end 132.562601 74.447399) (width 0.3048) (layer B.Cu) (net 22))
 (segment (start 74.93 101.6) (end 74.93 79.375) (width 0.3048) (layer B.Cu) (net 23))
 (segment (start 93.98 101.6) (end 93.98 79.375) (width 0.3048) (layer B.Cu) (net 24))
 (segment (start 112.242601 98.272601) (end 112.420399 98.094803) (width 0.3048) (layer B.Cu) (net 25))
 (segment (start 112.420399 98.094803) (end 112.420399 81.098152) (width 0.3048) (layer B.Cu) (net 25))
 (segment (start 112.420399 81.098152) (end 113.03 80.488551) (width 0.3048) (layer B.Cu) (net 25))
 (segment (start 113.03 80.488551) (end 113.03 79.375) (width 0.3048) (layer B.Cu) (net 25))
 (segment (start 113.03 101.6) (end 112.242601 100.812601) (width 0.3048) (layer B.Cu) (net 25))
 (segment (start 112.242601 100.812601) (end 112.242601 98.272601) (width 0.3048) (layer B.Cu) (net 25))
 (segment (start 132.08 79.375) (end 132.08 101.6) (width 0.3048) (layer B.Cu) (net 26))
 (via (at 107.315 110.669599) (size 1.5748) (drill 0.889) (layers F.Cu B.Cu) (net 11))
 (segment (start 101.180401 110.669599) (end 107.315 110.669599) (width 0.762) (layer F.Cu) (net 11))
 (segment (start 109.651799 90.373201) (end 109.651799 108.3328) (width 0.762) (layer B.Cu) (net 11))
 (segment (start 107.315 110.669599) (end 116.369599 110.669599) (width 0.762) (layer F.Cu) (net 11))
 (segment (start 109.651799 108.3328) (end 107.315 110.669599) (width 0.762) (layer B.Cu) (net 11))
 (segment (start 111.125 88.9) (end 109.651799 90.373201) (width 0.762) (layer B.Cu) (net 11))
 (segment (start 111.125 88.9) (end 113.665 88.9) (width 0.762) (layer F.Cu) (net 11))
 (segment (start 126.16 112.6) (end 128.090401 110.669599) (width 0.762) (layer F.Cu) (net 11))
 (segment (start 128.090401 110.669599) (end 135.419599 110.669599) (width 0.762) (layer F.Cu) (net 11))
 (segment (start 135.419599 110.669599) (end 136.562601 111.812601) (width 0.762) (layer F.Cu) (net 11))
 (segment (start 136.562601 111.812601) (end 137.35 112.6) (width 0.762) (layer F.Cu) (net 11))
 (segment (start 118.3 112.6) (end 126.16 112.6) (width 0.762) (layer F.Cu) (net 11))
 (segment (start 99.25 112.6) (end 101.180401 110.669599) (width 0.762) (layer F.Cu) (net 11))
 (segment (start 116.369599 110.669599) (end 117.512601 111.812601) (width 0.762) (layer F.Cu) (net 11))
 (segment (start 117.512601 111.812601) (end 118.3 112.6) (width 0.762) (layer F.Cu) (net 11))
 (segment (start 87.63 110.49) (end 97.14 110.49) (width 0.762) (layer F.Cu) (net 11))
 (segment (start 97.14 110.49) (end 98.462601 111.812601) (width 0.762) (layer F.Cu) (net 11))
 (segment (start 98.462601 111.812601) (end 99.25 112.6) (width 0.762) (layer F.Cu) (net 11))
 (segment (start 85.52 112.6) (end 87.63 110.49) (width 0.762) (layer F.Cu) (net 11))
 (segment (start 80.2 112.6) (end 85.52 112.6) (width 0.762) (layer F.Cu) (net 11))
 (segment (start 105.655529 87.198211) (end 105.24913 87.60461) (width 0.762) (layer F.Cu) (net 14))
 (segment (start 114.503211 87.198211) (end 105.655529 87.198211) (width 0.762) (layer F.Cu) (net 14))
 (segment (start 116.205 88.9) (end 114.503211 87.198211) (width 0.762) (layer F.Cu) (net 14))
 (segment (start 104.775 88.244031) (end 104.135579 87.60461) (width 0.762) (layer B.Cu) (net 14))
 (segment (start 104.775 108.55959) (end 104.775 88.244031) (width 0.762) (layer B.Cu) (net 14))
 (segment (start 105.24913 87.60461) (end 104.135579 87.60461) (width 0.762) (layer F.Cu) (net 14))
 (via (at 104.135579 87.60461) (size 1.5748) (drill 0.889) (layers F.Cu B.Cu) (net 14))
 (segment (start 91.44 108.55959) (end 104.775 108.55959) (width 0.762) (layer F.Cu) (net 14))
 (segment (start 104.775 108.55959) (end 110.464589 108.55959) (width 0.762) (layer F.Cu) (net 14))
 (via (at 104.775 108.55959) (size 1.5748) (drill 0.889) (layers F.Cu B.Cu) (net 14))
 (segment (start 110.464589 108.55959) (end 110.986516 109.081517) (width 0.762) (layer F.Cu) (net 14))
 (segment (start 111.33648 108.731553) (end 110.986516 109.081517) (width 0.762) (layer F.Cu) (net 14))
 (segment (start 110.3 112.6) (end 110.3 109.768033) (width 0.762) (layer B.Cu) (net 14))
 (segment (start 129.393447 108.731553) (end 111.33648 108.731553) (width 0.762) (layer F.Cu) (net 14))
 (via (at 110.986516 109.081517) (size 1.5748) (drill 0.889) (layers F.Cu B.Cu) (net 14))
 (segment (start 110.3 109.768033) (end 110.986516 109.081517) (width 0.762) (layer B.Cu) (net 14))
 (segment (start 129.35 108.775) (end 129.393447 108.731553) (width 0.762) (layer B.Cu) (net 14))
 (segment (start 129.35 112.6) (end 129.35 108.775) (width 0.762) (layer B.Cu) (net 14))
 (via (at 129.393447 108.731553) (size 1.5748) (drill 0.889) (layers F.Cu B.Cu) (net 14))
 (segment (start 116.205 88.9) (end 118.745 88.9) (width 0.762) (layer F.Cu) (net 14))
 (segment (start 76.24041 108.55959) (end 91.44 108.55959) (width 0.762) (layer F.Cu) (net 14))
 (segment (start 72.2 112.6) (end 76.24041 108.55959) (width 0.762) (layer F.Cu) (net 14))
 (segment (start 91.25 108.74959) (end 91.44 108.55959) (width 0.762) (layer B.Cu) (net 14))
 (segment (start 91.25 112.6) (end 91.25 108.74959) (width 0.762) (layer B.Cu) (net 14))
 (via (at 91.44 108.55959) (size 1.5748) (drill 0.889) (layers F.Cu B.Cu) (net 14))
 (segment (start 128.905 81.915) (end 128.905 69.933551) (width 0.762) (layer B.Cu) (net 17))
 (segment (start 128.905 69.933551) (end 129.35 69.488551) (width 0.762) (layer B.Cu) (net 17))
 (segment (start 129.35 69.488551) (end 129.35 68.375) (width 0.762) (layer B.Cu) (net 17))
 (segment (start 123.825 86.995) (end 128.905 81.915) (width 0.762) (layer B.Cu) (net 17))
 (segment (start 123.825 88.9) (end 123.825 86.995) (width 0.762) (layer B.Cu) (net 17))
 (segment (start 89.535 69.85) (end 73.675 69.85) (width 0.762) (layer F.Cu) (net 17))
 (segment (start 73.675 69.85) (end 72.2 68.375) (width 0.762) (layer F.Cu) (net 17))
 (segment (start 89.536799 69.848201) (end 89.535 69.85) (width 0.762) (layer F.Cu) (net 17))
 (segment (start 91.25 68.375) (end 89.776799 69.848201) (width 0.762) (layer F.Cu) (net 17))
 (segment (start 89.776799 69.848201) (end 89.536799 69.848201) (width 0.762) (layer F.Cu) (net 17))
 (segment (start 93.995 71.12) (end 91.25 68.375) (width 0.762) (layer F.Cu) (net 17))
 (segment (start 107.555 71.12) (end 93.995 71.12) (width 0.762) (layer F.Cu) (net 17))
 (segment (start 110.3 68.375) (end 107.555 71.12) (width 0.762) (layer F.Cu) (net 17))
 (segment (start 129.35 68.375) (end 127.24 70.485) (width 0.762) (layer F.Cu) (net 17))
 (segment (start 127.24 70.485) (end 112.41 70.485) (width 0.762) (layer F.Cu) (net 17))
 (segment (start 112.41 70.485) (end 110.3 68.375) (width 0.762) (layer F.Cu) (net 17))
 (segment (start 121.285 88.9) (end 123.825 88.9) (width 0.762) (layer F.Cu) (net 17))
 (segment (start 118.195982 72.59321) (end 118.680393 72.108799) (width 0.762) (layer F.Cu) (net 20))
 (segment (start 119.793944 72.108799) (end 118.680393 72.108799) (width 0.762) (layer F.Cu) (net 20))
 (segment (start 118.3 71.728406) (end 118.680393 72.108799) (width 0.762) (layer B.Cu) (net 20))
 (segment (start 118.3 68.375) (end 118.3 71.728406) (width 0.762) (layer B.Cu) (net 20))
 (segment (start 136.243799 72.108799) (end 119.793944 72.108799) (width 0.762) (layer F.Cu) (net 20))
 (segment (start 99.033351 72.59321) (end 118.195982 72.59321) (width 0.762) (layer F.Cu) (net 20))
 (segment (start 136.525 72.39) (end 136.243799 72.108799) (width 0.762) (layer F.Cu) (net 20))
 (via (at 118.680393 72.108799) (size 1.5748) (drill 0.889) (layers F.Cu B.Cu) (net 20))
 (segment (start 136.525 86.995) (end 136.525 72.39) (width 0.762) (layer F.Cu) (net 20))
 (segment (start 134.62 88.9) (end 136.525 86.995) (width 0.762) (layer F.Cu) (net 20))
 (segment (start 128.905 88.9) (end 134.62 88.9) (width 0.762) (layer F.Cu) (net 20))
 (segment (start 98.830141 72.39) (end 99.033351 72.59321) (width 0.762) (layer F.Cu) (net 20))
 (segment (start 80.01 72.39) (end 98.830141 72.39) (width 0.762) (layer F.Cu) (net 20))
 (segment (start 99.25 72.376561) (end 99.033351 72.59321) (width 0.762) (layer B.Cu) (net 20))
 (segment (start 99.25 68.375) (end 99.25 72.376561) (width 0.762) (layer B.Cu) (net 20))
 (via (at 99.033351 72.59321) (size 1.5748) (drill 0.889) (layers F.Cu B.Cu) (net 20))
 (segment (start 80.01 72.39) (end 80.01 68.565) (width 0.762) (layer B.Cu) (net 20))
 (segment (start 80.01 68.565) (end 80.2 68.375) (width 0.762) (layer B.Cu) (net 20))
 (via (at 80.01 72.39) (size 1.5748) (drill 0.889) (layers F.Cu B.Cu) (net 20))
 (segment (start 137.16 71.755) (end 136.525 72.39) (width 0.762) (layer F.Cu) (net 20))
 (segment (start 137.16 69.678551) (end 137.16 71.755) (width 0.762) (layer F.Cu) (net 20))
 (segment (start 137.35 68.375) (end 137.35 69.488551) (width 0.762) (layer F.Cu) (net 20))
 (segment (start 137.35 69.488551) (end 137.16 69.678551) (width 0.762) (layer F.Cu) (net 20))
 (segment (start 126.365 88.9) (end 128.905 88.9) (width 0.762) (layer F.Cu) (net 20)))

